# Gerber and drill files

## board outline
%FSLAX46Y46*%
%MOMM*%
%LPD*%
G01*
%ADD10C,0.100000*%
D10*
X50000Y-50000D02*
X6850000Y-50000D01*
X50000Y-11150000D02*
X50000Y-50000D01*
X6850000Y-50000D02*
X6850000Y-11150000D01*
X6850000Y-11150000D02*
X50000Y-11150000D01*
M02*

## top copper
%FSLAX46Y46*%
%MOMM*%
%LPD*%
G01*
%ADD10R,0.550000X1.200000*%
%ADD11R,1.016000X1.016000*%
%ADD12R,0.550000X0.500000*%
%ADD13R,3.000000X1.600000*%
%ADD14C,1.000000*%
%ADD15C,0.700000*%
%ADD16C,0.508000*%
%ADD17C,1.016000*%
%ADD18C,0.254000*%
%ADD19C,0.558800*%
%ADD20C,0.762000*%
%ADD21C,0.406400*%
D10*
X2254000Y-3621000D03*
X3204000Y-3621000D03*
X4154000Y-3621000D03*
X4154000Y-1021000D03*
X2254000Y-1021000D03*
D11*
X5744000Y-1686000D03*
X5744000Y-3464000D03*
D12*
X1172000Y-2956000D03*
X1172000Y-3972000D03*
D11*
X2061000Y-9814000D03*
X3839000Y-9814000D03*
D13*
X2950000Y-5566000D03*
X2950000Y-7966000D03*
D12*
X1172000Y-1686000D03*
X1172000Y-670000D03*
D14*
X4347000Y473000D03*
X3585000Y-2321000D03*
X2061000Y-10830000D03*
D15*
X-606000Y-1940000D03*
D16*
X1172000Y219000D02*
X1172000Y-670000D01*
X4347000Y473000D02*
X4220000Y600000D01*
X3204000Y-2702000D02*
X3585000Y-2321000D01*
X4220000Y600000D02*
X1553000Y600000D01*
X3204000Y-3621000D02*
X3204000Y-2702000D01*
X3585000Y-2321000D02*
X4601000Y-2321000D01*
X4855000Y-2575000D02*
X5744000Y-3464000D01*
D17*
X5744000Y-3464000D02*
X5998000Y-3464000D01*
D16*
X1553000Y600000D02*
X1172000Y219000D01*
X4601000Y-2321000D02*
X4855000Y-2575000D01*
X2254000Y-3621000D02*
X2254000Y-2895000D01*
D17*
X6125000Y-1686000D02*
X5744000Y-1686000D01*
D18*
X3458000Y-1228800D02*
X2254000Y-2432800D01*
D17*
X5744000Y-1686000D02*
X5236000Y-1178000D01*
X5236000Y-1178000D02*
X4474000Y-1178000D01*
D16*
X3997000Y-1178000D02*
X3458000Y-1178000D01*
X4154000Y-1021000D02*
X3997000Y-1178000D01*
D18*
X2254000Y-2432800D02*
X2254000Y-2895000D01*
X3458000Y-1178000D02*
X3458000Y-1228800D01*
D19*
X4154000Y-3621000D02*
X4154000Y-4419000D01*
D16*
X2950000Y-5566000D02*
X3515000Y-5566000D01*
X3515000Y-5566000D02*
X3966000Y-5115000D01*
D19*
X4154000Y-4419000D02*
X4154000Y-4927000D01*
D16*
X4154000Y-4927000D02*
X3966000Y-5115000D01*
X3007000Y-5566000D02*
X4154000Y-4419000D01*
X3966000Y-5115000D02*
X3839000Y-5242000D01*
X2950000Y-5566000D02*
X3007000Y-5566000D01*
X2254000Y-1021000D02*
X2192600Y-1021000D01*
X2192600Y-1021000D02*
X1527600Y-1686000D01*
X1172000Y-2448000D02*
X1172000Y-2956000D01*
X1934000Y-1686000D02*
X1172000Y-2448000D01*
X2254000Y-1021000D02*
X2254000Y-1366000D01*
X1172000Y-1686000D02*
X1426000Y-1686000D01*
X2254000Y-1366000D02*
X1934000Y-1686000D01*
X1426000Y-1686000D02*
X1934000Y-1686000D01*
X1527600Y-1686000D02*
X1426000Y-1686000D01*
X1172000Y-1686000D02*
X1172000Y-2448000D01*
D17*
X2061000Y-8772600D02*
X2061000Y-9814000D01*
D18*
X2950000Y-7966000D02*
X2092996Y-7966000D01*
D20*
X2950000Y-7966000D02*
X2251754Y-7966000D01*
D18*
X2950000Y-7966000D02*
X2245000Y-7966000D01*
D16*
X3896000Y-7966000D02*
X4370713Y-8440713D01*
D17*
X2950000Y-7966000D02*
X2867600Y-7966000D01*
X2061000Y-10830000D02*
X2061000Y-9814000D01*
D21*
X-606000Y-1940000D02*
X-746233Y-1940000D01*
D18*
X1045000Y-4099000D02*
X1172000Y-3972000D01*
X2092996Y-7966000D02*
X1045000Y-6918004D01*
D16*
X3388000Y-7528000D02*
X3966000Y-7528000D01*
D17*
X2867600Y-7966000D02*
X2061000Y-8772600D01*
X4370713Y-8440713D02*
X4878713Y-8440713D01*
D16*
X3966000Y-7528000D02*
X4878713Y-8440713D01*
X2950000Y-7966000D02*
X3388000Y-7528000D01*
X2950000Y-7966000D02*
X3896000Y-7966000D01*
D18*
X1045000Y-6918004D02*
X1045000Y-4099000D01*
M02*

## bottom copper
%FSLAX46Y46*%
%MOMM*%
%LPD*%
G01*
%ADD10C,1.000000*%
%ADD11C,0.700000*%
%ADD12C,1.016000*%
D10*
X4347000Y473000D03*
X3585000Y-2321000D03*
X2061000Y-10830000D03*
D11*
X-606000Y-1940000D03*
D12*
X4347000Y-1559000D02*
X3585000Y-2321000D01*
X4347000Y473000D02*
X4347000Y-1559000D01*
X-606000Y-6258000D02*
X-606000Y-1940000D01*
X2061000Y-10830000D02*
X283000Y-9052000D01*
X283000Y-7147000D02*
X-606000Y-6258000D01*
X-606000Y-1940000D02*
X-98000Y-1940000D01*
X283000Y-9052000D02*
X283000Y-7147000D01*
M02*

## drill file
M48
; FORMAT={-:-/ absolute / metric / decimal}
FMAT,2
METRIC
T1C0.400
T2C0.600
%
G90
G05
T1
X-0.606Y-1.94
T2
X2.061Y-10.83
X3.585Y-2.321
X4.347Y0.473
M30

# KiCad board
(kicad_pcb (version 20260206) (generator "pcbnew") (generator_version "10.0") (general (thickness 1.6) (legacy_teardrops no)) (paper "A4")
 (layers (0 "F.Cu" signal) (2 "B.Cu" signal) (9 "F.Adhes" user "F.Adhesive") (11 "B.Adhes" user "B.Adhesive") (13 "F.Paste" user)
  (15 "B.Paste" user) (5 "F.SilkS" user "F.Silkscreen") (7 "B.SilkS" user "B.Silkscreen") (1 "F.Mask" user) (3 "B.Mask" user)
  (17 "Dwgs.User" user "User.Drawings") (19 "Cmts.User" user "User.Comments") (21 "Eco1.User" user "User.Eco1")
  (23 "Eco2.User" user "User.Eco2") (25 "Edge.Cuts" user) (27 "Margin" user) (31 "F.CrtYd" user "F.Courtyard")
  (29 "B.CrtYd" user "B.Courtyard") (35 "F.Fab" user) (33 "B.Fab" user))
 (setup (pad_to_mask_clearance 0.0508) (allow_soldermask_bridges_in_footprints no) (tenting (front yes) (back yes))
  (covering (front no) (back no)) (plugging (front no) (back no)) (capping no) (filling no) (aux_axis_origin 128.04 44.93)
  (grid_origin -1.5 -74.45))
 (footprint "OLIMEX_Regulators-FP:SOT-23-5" (layer "F.Cu") (at 3.204 2.321 -90)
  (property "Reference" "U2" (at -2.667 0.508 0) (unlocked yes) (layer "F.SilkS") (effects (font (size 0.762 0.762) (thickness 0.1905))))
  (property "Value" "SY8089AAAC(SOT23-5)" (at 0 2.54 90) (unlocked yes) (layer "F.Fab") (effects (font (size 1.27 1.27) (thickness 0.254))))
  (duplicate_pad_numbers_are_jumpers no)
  (pad "1" smd rect (at 1.3 0.95 270) (size 1.2 0.55) (layers "F.Cu" "F.Mask" "F.Paste") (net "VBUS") (solder_mask_margin 0.0508)
   (clearance 0.0508))
  (pad "2" smd rect (at 1.3 0 270) (size 1.2 0.55) (layers "F.Cu" "F.Mask" "F.Paste") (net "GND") (solder_mask_margin 0.0508)
   (clearance 0.0508))
  (pad "3" smd rect (at 1.3 -0.95 270) (size 1.2 0.55) (layers "F.Cu" "F.Mask" "F.Paste") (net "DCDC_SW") (solder_mask_margin 0.0508)
   (clearance 0.0508))
  (pad "4" smd rect (at -1.3 -0.95 270) (size 1.2 0.55) (layers "F.Cu" "F.Mask" "F.Paste") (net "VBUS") (solder_mask_margin 0.0508)
   (clearance 0.0508))
  (pad "5" smd rect (at -1.3 0.95 270) (size 1.2 0.55) (layers "F.Cu" "F.Mask" "F.Paste") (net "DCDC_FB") (solder_mask_margin 0.0508)
   (clearance 0.0508)))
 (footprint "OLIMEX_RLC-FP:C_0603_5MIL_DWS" (layer "F.Cu") (at 5.744 2.575 -90)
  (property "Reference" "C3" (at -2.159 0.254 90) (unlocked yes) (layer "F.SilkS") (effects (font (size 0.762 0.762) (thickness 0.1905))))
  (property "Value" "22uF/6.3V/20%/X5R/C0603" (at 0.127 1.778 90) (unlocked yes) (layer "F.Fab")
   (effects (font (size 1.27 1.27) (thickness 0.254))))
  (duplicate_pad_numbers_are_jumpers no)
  (pad "1" smd rect (at -0.889 0 270) (size 1.016 1.016) (layers "F.Cu" "F.Mask" "F.Paste") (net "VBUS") (solder_mask_margin 0.0508)
   (clearance 0.0508))
  (pad "2" smd rect (at 0.889 0 270) (size 1.016 1.016) (layers "F.Cu" "F.Mask" "F.Paste") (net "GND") (solder_mask_margin 0.0508)
   (clearance 0.0508)))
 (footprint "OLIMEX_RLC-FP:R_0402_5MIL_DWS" (layer "F.Cu") (at 1.172 3.464 -90)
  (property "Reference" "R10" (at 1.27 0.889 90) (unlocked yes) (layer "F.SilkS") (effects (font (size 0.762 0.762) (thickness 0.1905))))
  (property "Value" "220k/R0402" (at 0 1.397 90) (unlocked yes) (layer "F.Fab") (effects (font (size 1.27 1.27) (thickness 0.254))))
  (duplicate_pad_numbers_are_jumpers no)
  (pad "1" smd rect (at -0.508 0 90) (size 0.5 0.55) (layers "F.Cu" "F.Mask" "F.Paste") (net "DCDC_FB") (solder_mask_margin 0.0508))
  (pad "2" smd rect (at 0.508 0 270) (size 0.5 0.55) (layers "F.Cu" "F.Mask" "F.Paste") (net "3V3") (solder_mask_margin 0.0508)))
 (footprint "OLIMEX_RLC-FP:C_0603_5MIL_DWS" (layer "F.Cu") (at 2.95 9.814)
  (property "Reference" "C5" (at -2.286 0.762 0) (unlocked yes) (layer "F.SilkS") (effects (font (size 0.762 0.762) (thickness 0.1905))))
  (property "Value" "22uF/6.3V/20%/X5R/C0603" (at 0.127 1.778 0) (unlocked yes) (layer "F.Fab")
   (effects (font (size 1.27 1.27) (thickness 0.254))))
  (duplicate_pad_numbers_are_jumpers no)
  (pad "1" smd rect (at -0.889 0) (size 1.016 1.016) (layers "F.Cu" "F.Mask" "F.Paste") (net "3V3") (solder_mask_margin 0.0508)
   (clearance 0.0508))
  (pad "2" smd rect (at 0.889 0) (size 1.016 1.016) (layers "F.Cu" "F.Mask" "F.Paste") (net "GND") (solder_mask_margin 0.0508)
   (clearance 0.0508)))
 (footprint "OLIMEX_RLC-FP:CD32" (layer "F.Cu") (at 2.95 6.766 -90)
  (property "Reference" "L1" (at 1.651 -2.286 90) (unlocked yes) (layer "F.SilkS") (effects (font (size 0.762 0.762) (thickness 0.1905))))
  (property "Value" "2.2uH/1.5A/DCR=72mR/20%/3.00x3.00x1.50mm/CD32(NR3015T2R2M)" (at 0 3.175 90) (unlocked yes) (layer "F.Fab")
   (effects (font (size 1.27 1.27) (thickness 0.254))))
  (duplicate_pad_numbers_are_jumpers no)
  (pad "1" smd rect (at -1.2 0 90) (size 1.6 3) (layers "F.Cu" "F.Mask" "F.Paste") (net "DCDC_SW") (solder_mask_margin 0.0508)
   (clearance 0.0508))
  (pad "2" smd rect (at 1.2 0 90) (size 1.6 3) (layers "F.Cu" "F.Mask" "F.Paste") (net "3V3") (solder_mask_margin 0.0508) (clearance 0.0508)))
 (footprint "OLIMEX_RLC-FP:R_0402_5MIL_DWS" (layer "F.Cu") (at 1.172 1.178 90)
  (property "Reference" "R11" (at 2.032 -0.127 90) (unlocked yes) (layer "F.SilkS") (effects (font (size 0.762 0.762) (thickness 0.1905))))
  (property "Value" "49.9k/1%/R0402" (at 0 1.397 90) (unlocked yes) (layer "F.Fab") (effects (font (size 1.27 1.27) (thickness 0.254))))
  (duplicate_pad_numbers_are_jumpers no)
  (pad "1" smd rect (at -0.508 0 270) (size 0.5 0.55) (layers "F.Cu" "F.Mask" "F.Paste") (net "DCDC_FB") (solder_mask_margin 0.0508))
  (pad "2" smd rect (at 0.508 0 90) (size 0.5 0.55) (layers "F.Cu" "F.Mask" "F.Paste") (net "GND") (solder_mask_margin 0.0508)))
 (gr_line (start 0.05 0.05) (end 6.85 0.05) (stroke (width 0.1) (type default)) (layer "Edge.Cuts"))
 (gr_line (start 0.05 11.15) (end 0.05 0.05) (stroke (width 0.1) (type default)) (layer "Edge.Cuts"))
 (gr_line (start 6.85 0.05) (end 6.85 11.15) (stroke (width 0.1) (type default)) (layer "Edge.Cuts"))
 (gr_line (start 6.85 11.15) (end 0.05 11.15) (stroke (width 0.1) (type default)) (layer "Edge.Cuts"))
 (segment (start 1.172 -0.219) (end 1.172 0.67) (width 0.508) (layer "F.Cu") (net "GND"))
 (segment (start 4.347 -0.473) (end 4.22 -0.6) (width 0.508) (layer "F.Cu") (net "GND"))
 (segment (start 3.204 2.702) (end 3.585 2.321) (width 0.508) (layer "F.Cu") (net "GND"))
 (segment (start 4.22 -0.6) (end 1.553 -0.6) (width 0.508) (layer "F.Cu") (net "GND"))
 (segment (start 3.204 3.621) (end 3.204 2.702) (width 0.508) (layer "F.Cu") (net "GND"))
 (segment (start 3.585 2.321) (end 4.601 2.321) (width 0.508) (layer "F.Cu") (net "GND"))
 (segment (start 4.855 2.575) (end 5.744 3.464) (width 0.508) (layer "F.Cu") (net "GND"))
 (segment (start 5.744 3.464) (end 5.998 3.464) (width 1.016) (layer "F.Cu") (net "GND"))
 (segment (start 1.553 -0.6) (end 1.172 -0.219) (width 0.508) (layer "F.Cu") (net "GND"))
 (segment (start 4.601 2.321) (end 4.855 2.575) (width 0.508) (layer "F.Cu") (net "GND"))
 (via (at 4.347 -0.473) (size 1) (drill 0.6) (layers "F.Cu" "B.Cu") (capping no) (covering (front no) (back no))
  (plugging (front no) (back no)) (filling no) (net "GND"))
 (via (at 3.585 2.321) (size 1) (drill 0.6) (layers "F.Cu" "B.Cu") (capping no) (covering (front no) (back no))
  (plugging (front no) (back no)) (filling no) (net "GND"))
 (segment (start 4.347 1.559) (end 3.585 2.321) (width 1.016) (layer "B.Cu") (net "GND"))
 (segment (start 4.347 -0.473) (end 4.347 1.559) (width 1.016) (layer "B.Cu") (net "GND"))
 (segment (start 2.254 3.621) (end 2.254 2.895) (width 0.508) (layer "F.Cu") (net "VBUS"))
 (segment (start 6.125 1.686) (end 5.744 1.686) (width 1.016) (layer "F.Cu") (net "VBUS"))
 (segment (start 3.458 1.2288) (end 2.254 2.4328) (width 0.254) (layer "F.Cu") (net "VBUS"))
 (segment (start 5.744 1.686) (end 5.236 1.178) (width 1.016) (layer "F.Cu") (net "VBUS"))
 (segment (start 5.236 1.178) (end 4.474 1.178) (width 1.016) (layer "F.Cu") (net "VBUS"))
 (segment (start 3.997 1.178) (end 3.458 1.178) (width 0.508) (layer "F.Cu") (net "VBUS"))
 (segment (start 4.154 1.021) (end 3.997 1.178) (width 0.508) (layer "F.Cu") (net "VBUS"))
 (segment (start 2.254 2.4328) (end 2.254 2.895) (width 0.254) (layer "F.Cu") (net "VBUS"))
 (segment (start 3.458 1.178) (end 3.458 1.2288) (width 0.254) (layer "F.Cu") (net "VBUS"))
 (segment (start 4.154 3.621) (end 4.154 4.419) (width 0.5588) (layer "F.Cu") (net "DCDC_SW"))
 (segment (start 2.95 5.566) (end 3.515 5.566) (width 0.508) (layer "F.Cu") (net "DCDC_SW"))
 (segment (start 3.515 5.566) (end 3.966 5.115) (width 0.508) (layer "F.Cu") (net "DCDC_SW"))
 (segment (start 4.154 4.419) (end 4.154 4.927) (width 0.5588) (layer "F.Cu") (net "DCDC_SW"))
 (segment (start 4.154 4.927) (end 3.966 5.115) (width 0.508) (layer "F.Cu") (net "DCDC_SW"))
 (segment (start 3.007 5.566) (end 4.154 4.419) (width 0.508) (layer "F.Cu") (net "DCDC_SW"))
 (segment (start 3.966 5.115) (end 3.839 5.242) (width 0.508) (layer "F.Cu") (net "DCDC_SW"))
 (segment (start 2.95 5.566) (end 3.007 5.566) (width 0.508) (layer "F.Cu") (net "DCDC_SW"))
 (segment (start 2.254 1.021) (end 2.1926 1.021) (width 0.508) (layer "F.Cu") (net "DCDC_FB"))
 (segment (start 2.1926 1.021) (end 1.5276 1.686) (width 0.508) (layer "F.Cu") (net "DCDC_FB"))
 (segment (start 1.172 2.448) (end 1.172 2.956) (width 0.508) (layer "F.Cu") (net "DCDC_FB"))
 (segment (start 1.934 1.686) (end 1.172 2.448) (width 0.508) (layer "F.Cu") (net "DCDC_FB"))
 (segment (start 2.254 1.021) (end 2.254 1.366) (width 0.508) (layer "F.Cu") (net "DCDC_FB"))
 (segment (start 1.172 1.686) (end 1.426 1.686) (width 0.508) (layer "F.Cu") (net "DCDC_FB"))
 (segment (start 2.254 1.366) (end 1.934 1.686) (width 0.508) (layer "F.Cu") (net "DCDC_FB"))
 (segment (start 1.426 1.686) (end 1.934 1.686) (width 0.508) (layer "F.Cu") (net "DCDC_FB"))
 (segment (start 1.5276 1.686) (end 1.426 1.686) (width 0.508) (layer "F.Cu") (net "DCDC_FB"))
 (segment (start 1.172 1.686) (end 1.172 2.448) (width 0.508) (layer "F.Cu") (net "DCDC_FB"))
 (segment (start 2.061 8.7726) (end 2.061 9.814) (width 1.016) (layer "F.Cu") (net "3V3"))
 (segment (start 2.95 7.966) (end 2.092996 7.966) (width 0.254) (layer "F.Cu") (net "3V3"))
 (segment (start 2.95 7.966) (end 2.251754 7.966) (width 0.762) (layer "F.Cu") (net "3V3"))
 (segment (start 2.95 7.966) (end 2.245 7.966) (width 0.254) (layer "F.Cu") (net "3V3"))
 (segment (start 3.896 7.966) (end 4.370713 8.440713) (width 0.508) (layer "F.Cu") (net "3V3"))
 (segment (start 2.95 7.966) (end 2.8676 7.966) (width 1.016) (layer "F.Cu") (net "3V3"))
 (segment (start 2.061 10.83) (end 2.061 9.814) (width 1.016) (layer "F.Cu") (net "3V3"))
 (segment (start -0.606 1.94) (end -0.746233 1.94) (width 0.4064) (layer "F.Cu") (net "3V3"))
 (segment (start 1.045 4.099) (end 1.172 3.972) (width 0.254) (layer "F.Cu") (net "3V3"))
 (segment (start 2.092996 7.966) (end 1.045 6.918004) (width 0.254) (layer "F.Cu") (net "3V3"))
 (segment (start 3.388 7.528) (end 3.966 7.528) (width 0.508) (layer "F.Cu") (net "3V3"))
 (segment (start 2.8676 7.966) (end 2.061 8.7726) (width 1.016) (layer "F.Cu") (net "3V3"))
 (segment (start 4.370713 8.440713) (end 4.878713 8.440713) (width 1.016) (layer "F.Cu") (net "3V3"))
 (segment (start 3.966 7.528) (end 4.878713 8.440713) (width 0.508) (layer "F.Cu") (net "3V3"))
 (segment (start 2.95 7.966) (end 3.388 7.528) (width 0.508) (layer "F.Cu") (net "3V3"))
 (segment (start 2.95 7.966) (end 3.896 7.966) (width 0.508) (layer "F.Cu") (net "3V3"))
 (segment (start 1.045 6.918004) (end 1.045 4.099) (width 0.254) (layer "F.Cu") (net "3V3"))
 (via (at 2.061 10.83) (size 1) (drill 0.6) (layers "F.Cu" "B.Cu") (capping no) (covering (front no) (back no))
  (plugging (front no) (back no)) (filling no) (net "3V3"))
 (via (at -0.606 1.94) (size 0.7) (drill 0.4) (layers "F.Cu" "B.Cu") (capping no) (covering (front no) (back no))
  (plugging (front no) (back no)) (filling no) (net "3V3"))
 (segment (start -0.606 6.258) (end -0.606 1.94) (width 1.016) (layer "B.Cu") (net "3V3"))
 (segment (start 2.061 10.83) (end 0.283 9.052) (width 1.016) (layer "B.Cu") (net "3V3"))
 (segment (start 0.283 7.147) (end -0.606 6.258) (width 1.016) (layer "B.Cu") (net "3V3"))
 (segment (start -0.606 1.94) (end -0.098 1.94) (width 1.016) (layer "B.Cu") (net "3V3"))
 (segment (start 0.283 9.052) (end 0.283 7.147) (width 1.016) (layer "B.Cu") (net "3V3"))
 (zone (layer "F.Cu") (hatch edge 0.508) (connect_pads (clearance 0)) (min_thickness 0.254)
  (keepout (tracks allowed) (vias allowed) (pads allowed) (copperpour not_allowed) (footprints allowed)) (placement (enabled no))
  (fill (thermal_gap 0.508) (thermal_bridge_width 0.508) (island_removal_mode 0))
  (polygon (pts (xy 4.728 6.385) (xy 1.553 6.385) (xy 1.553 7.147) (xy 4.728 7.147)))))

